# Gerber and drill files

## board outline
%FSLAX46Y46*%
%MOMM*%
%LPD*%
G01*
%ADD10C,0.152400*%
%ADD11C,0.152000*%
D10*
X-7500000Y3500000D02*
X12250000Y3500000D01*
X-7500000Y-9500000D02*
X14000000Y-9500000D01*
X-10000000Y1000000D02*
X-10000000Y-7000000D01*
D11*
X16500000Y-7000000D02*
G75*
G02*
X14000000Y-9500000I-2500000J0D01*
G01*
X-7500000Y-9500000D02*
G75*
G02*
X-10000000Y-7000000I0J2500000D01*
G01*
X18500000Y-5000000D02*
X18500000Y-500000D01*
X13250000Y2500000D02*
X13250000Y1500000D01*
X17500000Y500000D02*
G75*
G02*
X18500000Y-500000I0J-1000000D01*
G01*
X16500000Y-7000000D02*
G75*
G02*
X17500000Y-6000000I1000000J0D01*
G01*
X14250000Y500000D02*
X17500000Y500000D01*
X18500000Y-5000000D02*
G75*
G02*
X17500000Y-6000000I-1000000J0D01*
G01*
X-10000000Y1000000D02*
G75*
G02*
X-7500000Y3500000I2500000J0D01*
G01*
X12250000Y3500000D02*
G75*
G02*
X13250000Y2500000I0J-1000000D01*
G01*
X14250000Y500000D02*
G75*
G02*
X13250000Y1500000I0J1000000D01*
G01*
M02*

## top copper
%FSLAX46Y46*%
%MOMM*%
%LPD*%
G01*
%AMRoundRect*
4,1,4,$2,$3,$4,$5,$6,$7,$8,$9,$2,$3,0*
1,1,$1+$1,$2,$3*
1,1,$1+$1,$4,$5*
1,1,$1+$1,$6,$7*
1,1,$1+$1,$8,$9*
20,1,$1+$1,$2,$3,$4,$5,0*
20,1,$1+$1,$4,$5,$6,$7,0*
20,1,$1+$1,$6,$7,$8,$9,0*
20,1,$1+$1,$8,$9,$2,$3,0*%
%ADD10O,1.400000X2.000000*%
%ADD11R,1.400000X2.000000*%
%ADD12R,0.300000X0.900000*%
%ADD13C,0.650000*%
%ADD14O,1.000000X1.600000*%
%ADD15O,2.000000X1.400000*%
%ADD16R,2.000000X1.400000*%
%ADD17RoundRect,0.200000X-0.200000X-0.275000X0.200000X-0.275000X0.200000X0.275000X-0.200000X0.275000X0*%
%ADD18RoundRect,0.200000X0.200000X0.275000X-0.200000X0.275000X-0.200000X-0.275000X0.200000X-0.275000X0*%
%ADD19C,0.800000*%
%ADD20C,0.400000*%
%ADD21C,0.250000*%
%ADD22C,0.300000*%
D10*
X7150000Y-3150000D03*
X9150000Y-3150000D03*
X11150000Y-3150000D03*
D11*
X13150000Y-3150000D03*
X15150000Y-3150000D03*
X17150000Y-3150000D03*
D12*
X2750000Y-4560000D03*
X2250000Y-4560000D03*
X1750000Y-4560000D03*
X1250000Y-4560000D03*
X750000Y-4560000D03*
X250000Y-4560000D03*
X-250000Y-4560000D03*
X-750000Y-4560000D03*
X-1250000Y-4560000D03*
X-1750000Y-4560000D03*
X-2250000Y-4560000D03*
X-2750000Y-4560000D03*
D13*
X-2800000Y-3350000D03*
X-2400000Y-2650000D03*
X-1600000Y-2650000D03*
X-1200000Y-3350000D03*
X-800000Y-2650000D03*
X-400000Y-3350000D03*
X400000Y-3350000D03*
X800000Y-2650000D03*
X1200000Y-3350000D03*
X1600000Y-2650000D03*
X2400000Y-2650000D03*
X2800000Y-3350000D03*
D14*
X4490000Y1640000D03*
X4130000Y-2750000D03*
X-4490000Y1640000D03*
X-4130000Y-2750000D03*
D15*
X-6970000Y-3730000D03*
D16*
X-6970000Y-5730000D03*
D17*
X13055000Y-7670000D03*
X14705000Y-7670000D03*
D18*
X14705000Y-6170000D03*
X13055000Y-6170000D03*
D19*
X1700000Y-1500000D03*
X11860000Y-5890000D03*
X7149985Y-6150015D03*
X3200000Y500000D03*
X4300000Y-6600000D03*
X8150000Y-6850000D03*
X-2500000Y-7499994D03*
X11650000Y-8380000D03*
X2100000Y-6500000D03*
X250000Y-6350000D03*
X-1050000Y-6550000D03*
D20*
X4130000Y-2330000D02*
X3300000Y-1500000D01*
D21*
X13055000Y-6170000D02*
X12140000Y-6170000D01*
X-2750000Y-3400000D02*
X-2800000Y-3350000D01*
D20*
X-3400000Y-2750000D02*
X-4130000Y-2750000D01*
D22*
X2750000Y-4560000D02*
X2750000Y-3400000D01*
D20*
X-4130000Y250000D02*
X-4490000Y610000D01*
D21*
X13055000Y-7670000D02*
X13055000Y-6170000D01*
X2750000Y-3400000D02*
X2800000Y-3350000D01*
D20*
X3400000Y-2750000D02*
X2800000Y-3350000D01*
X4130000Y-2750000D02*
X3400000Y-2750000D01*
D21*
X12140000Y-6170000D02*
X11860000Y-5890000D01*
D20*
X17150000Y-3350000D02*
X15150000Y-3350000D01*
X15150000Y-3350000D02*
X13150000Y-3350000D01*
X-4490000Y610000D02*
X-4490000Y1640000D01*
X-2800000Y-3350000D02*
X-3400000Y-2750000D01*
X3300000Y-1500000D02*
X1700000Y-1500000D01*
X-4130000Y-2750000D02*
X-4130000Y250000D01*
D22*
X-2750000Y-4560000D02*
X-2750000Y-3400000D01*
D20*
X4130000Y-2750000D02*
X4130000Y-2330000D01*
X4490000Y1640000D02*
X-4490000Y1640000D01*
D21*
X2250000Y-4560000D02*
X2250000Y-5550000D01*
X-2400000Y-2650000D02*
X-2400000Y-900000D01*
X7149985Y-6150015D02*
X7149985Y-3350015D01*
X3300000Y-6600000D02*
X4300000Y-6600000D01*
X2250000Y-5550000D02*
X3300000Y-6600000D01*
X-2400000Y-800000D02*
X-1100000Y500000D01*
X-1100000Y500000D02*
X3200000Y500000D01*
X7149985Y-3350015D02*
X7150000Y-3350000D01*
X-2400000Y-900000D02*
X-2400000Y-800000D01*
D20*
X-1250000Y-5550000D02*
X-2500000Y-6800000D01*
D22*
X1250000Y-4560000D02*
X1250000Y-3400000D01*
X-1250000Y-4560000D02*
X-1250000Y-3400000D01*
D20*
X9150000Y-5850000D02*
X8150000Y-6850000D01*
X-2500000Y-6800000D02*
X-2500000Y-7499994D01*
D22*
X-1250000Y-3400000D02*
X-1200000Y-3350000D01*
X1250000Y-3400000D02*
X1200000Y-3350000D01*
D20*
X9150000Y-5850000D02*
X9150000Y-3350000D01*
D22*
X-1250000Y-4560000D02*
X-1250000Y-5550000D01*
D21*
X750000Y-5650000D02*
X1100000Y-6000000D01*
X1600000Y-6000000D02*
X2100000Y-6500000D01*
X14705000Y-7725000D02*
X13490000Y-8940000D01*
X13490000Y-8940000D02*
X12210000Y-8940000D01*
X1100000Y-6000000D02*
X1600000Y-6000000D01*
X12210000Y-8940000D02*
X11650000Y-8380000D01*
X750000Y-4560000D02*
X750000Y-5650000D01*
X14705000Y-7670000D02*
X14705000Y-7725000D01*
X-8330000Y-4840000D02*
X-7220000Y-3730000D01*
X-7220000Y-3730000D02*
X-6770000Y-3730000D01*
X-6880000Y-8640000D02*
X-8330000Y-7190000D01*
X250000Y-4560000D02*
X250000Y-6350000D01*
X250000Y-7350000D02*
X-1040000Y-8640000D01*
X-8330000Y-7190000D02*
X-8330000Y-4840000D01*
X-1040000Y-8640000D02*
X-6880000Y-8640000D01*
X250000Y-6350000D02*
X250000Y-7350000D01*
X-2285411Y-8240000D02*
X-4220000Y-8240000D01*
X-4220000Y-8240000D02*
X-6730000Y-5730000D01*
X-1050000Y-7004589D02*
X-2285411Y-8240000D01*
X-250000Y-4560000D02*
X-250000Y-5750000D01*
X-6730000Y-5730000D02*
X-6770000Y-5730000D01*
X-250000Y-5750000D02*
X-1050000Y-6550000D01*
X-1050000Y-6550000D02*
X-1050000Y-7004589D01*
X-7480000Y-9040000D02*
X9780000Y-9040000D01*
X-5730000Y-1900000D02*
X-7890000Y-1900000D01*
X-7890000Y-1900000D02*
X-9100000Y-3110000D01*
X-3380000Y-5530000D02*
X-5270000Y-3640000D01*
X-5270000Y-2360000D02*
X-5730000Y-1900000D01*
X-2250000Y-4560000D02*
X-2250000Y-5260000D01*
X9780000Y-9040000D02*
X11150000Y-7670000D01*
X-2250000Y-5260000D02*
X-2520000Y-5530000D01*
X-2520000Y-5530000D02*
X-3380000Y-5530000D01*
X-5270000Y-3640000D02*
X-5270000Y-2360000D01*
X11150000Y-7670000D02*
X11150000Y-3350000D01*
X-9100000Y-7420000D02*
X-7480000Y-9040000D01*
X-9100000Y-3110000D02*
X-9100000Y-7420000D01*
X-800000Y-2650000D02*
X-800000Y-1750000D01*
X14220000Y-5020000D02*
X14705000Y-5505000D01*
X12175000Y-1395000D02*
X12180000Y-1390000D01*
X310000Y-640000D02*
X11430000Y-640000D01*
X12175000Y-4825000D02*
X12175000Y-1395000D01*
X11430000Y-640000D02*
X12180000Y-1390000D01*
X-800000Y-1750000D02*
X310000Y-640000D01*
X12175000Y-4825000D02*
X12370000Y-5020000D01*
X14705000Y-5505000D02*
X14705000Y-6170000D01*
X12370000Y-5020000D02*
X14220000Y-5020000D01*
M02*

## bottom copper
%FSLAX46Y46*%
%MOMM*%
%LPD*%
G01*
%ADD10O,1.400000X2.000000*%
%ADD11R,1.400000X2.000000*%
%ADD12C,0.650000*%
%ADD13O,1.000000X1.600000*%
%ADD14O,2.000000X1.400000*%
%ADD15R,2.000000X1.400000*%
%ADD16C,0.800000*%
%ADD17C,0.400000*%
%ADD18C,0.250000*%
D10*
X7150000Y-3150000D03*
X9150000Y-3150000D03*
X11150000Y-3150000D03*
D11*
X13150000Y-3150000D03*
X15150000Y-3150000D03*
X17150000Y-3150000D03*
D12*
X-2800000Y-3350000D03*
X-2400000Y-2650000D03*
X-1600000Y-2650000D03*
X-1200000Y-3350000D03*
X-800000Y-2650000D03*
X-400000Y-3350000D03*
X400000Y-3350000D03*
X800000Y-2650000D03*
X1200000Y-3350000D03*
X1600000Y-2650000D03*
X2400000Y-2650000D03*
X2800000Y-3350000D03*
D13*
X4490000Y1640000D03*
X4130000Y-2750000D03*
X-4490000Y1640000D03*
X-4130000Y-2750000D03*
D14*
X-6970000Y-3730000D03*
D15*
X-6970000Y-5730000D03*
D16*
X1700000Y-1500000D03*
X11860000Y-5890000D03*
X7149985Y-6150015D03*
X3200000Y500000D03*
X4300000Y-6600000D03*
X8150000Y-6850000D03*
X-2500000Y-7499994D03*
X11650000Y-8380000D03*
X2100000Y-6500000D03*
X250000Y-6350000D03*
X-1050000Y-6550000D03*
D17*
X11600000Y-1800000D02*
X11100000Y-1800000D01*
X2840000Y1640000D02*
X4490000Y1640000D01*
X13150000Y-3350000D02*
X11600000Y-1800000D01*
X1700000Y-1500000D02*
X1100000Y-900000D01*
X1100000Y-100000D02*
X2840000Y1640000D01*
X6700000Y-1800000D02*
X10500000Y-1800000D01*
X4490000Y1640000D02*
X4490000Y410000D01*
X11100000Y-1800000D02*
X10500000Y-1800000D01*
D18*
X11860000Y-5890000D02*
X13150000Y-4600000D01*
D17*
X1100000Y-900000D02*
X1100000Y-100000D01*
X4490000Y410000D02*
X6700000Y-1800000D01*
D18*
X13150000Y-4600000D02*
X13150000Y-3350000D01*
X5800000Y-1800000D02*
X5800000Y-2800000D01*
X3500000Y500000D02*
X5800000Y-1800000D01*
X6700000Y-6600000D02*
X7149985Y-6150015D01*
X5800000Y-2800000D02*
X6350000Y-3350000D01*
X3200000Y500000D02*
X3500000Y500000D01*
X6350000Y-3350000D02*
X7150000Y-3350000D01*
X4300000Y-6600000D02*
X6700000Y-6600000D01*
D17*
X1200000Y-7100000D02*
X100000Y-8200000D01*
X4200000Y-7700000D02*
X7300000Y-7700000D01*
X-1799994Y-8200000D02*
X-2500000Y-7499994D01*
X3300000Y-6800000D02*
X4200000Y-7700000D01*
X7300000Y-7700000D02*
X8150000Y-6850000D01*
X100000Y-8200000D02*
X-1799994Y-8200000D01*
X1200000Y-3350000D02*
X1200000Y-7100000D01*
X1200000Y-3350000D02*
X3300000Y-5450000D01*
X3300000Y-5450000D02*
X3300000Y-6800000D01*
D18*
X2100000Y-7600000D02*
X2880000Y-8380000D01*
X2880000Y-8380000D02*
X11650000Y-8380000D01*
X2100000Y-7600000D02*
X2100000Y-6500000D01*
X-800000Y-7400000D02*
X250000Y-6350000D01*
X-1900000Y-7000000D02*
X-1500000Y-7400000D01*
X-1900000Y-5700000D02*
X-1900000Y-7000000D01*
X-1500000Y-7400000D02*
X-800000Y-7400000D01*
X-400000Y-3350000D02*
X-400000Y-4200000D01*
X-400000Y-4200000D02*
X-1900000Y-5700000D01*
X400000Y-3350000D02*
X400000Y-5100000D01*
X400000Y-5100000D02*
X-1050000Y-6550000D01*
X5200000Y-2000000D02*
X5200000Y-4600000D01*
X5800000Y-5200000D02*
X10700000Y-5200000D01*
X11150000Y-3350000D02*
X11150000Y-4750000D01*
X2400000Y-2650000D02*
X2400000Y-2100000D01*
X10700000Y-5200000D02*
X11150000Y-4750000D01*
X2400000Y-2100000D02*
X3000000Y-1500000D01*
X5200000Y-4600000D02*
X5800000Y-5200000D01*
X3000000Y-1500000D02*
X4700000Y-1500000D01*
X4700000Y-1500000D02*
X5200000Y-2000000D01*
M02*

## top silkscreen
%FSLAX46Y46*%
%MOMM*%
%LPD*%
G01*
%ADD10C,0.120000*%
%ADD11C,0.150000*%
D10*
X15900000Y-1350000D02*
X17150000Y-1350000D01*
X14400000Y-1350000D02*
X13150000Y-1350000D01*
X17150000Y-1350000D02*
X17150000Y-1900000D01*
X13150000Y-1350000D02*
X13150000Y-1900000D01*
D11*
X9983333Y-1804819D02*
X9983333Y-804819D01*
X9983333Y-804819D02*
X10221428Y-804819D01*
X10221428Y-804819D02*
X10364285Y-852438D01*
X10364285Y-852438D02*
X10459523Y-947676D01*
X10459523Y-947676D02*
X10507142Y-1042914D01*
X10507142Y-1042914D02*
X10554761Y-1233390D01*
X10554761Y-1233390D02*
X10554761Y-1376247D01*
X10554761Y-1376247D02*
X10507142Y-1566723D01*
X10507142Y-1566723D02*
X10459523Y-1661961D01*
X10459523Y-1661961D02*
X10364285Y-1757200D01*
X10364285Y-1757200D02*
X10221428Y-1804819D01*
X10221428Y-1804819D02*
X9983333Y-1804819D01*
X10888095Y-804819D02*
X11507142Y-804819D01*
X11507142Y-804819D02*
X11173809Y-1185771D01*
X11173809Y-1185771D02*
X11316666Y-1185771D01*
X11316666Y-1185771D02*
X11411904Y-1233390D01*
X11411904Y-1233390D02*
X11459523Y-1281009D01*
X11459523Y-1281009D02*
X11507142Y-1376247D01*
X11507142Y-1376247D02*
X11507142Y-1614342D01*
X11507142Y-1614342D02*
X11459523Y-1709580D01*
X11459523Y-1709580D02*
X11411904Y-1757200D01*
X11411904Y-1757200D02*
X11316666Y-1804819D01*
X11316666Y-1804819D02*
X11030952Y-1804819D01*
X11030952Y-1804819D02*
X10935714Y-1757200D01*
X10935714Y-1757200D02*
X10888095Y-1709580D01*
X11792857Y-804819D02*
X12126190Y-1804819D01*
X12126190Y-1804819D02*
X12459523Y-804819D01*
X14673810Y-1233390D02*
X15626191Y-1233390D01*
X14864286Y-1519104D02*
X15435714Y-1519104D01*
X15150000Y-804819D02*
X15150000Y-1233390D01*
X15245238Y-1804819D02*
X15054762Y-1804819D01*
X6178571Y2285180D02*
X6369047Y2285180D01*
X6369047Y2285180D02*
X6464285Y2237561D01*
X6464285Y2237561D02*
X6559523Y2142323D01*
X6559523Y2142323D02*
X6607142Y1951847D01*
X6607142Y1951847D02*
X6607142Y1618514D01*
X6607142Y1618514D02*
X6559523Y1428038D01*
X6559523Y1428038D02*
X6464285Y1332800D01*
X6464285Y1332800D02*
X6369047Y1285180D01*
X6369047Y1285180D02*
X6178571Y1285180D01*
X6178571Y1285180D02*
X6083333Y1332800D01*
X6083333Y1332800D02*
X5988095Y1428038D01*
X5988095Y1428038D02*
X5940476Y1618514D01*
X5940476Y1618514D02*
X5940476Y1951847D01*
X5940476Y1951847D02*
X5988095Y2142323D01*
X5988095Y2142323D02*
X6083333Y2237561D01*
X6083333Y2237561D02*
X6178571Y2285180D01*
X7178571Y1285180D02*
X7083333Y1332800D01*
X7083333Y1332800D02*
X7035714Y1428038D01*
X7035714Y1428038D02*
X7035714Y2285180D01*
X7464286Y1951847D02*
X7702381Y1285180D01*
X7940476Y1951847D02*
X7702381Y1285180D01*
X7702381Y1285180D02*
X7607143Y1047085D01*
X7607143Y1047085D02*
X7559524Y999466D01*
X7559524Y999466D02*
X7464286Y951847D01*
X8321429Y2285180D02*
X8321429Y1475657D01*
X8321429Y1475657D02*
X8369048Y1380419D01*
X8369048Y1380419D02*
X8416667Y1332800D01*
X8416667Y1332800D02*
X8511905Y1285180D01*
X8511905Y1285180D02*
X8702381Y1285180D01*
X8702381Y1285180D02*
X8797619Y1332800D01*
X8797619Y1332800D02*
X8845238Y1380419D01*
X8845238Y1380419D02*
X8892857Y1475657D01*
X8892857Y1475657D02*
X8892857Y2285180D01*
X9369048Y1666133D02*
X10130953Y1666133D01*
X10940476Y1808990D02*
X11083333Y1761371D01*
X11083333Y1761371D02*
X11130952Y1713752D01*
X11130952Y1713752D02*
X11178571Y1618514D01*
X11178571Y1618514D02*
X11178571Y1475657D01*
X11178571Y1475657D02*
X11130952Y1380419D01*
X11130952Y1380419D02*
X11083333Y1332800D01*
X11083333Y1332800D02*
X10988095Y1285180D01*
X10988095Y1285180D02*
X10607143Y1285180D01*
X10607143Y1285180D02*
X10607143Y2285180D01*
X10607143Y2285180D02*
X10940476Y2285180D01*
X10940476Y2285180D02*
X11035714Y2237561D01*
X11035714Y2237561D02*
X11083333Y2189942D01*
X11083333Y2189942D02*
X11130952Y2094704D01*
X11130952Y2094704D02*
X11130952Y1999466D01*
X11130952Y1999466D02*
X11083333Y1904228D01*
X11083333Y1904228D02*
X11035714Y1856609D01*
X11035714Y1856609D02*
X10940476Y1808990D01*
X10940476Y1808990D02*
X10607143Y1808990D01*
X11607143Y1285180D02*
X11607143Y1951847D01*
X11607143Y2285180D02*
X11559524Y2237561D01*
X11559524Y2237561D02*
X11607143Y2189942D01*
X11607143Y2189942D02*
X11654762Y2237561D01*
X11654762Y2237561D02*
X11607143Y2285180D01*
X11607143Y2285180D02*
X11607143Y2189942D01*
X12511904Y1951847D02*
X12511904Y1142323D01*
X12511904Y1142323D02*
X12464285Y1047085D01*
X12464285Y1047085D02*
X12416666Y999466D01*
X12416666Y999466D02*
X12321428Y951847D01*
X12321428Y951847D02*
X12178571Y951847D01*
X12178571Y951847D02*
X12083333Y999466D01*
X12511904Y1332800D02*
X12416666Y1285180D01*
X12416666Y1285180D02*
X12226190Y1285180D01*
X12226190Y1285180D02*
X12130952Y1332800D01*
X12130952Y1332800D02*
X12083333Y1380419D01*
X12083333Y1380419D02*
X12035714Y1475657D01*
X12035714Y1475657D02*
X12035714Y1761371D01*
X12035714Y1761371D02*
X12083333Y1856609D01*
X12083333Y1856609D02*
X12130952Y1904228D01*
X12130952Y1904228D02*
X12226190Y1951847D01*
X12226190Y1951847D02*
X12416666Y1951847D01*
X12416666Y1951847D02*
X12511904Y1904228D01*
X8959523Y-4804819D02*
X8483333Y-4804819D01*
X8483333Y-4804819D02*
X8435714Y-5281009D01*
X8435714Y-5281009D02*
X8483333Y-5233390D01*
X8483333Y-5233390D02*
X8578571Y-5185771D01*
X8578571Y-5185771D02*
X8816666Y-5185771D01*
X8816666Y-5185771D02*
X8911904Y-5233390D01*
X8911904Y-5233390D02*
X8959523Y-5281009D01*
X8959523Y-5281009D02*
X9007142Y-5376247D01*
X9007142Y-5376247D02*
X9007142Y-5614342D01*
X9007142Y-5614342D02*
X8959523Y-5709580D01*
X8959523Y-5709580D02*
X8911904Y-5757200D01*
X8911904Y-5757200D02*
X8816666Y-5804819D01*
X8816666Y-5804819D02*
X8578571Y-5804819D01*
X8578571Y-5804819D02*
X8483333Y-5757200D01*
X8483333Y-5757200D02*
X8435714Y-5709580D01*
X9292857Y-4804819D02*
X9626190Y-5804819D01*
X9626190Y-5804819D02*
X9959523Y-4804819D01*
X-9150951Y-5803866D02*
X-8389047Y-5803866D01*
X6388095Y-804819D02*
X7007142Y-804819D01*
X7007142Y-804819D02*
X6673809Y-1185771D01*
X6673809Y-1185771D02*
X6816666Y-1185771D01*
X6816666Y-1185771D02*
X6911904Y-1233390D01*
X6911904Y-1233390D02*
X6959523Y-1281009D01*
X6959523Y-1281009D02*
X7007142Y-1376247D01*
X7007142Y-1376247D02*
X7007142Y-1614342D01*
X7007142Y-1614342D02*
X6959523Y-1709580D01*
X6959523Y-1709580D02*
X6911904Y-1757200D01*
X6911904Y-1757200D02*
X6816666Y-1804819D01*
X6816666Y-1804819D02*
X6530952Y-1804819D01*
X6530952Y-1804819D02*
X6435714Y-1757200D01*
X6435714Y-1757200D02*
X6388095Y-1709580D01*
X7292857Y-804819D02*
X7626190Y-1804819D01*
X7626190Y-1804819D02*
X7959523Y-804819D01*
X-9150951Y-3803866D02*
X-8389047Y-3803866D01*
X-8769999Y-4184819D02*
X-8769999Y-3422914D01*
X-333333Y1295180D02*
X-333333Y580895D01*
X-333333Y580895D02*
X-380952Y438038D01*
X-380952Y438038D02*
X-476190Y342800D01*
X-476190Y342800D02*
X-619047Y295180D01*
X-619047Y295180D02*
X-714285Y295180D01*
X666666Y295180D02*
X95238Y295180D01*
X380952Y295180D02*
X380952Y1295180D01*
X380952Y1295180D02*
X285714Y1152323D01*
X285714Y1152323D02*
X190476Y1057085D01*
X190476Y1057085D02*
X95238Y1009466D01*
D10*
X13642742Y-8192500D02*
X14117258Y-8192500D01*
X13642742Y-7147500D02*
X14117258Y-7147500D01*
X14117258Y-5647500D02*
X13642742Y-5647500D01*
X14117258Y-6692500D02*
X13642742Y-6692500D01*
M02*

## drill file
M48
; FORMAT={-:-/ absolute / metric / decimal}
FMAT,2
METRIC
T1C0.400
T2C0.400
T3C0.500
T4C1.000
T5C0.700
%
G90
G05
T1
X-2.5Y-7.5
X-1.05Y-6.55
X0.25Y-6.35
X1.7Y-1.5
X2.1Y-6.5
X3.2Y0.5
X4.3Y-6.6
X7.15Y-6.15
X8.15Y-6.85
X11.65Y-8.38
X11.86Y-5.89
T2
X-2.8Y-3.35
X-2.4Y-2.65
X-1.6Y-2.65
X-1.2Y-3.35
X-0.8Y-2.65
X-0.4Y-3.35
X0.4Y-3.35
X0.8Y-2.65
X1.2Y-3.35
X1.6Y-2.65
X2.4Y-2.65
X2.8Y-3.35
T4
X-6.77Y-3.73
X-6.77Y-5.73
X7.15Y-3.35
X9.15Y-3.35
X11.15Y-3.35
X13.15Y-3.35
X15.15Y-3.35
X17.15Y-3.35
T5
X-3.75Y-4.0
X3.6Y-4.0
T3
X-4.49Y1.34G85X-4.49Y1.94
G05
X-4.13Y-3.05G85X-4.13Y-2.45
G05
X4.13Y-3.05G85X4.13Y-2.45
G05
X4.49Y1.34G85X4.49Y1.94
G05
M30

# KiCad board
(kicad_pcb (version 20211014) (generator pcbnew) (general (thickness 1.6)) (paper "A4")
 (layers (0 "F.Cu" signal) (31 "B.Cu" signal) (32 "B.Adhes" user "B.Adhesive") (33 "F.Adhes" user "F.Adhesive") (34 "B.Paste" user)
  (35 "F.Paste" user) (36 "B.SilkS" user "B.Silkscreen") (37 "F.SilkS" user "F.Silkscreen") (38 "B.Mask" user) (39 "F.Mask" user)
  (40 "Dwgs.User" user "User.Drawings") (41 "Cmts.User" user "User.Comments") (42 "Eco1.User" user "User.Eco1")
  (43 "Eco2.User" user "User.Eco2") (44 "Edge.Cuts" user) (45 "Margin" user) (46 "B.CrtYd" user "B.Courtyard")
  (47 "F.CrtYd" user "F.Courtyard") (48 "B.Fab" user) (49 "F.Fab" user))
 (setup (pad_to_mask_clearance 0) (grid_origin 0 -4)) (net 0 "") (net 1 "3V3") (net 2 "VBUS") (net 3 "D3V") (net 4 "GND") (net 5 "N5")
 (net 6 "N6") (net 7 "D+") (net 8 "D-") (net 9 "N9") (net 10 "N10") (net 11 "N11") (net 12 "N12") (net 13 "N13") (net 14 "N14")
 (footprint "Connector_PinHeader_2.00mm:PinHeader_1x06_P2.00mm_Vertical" (layer "F.Cu") (at 7.15 3.35 90)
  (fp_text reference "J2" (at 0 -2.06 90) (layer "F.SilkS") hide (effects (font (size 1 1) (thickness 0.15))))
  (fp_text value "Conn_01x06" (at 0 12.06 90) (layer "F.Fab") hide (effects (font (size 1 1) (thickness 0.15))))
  (pad "1" thru_hole oval locked (at 0 0 90) (size 2 1.4) (drill 1 (offset 0.2 0)) (layers *.Cu *.Mask) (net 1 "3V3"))
  (pad "2" thru_hole oval locked (at 0 2 90) (size 2 1.4) (drill 1 (offset 0.2 0)) (layers *.Cu *.Mask) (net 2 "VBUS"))
  (pad "3" thru_hole oval locked (at 0 4 90) (size 2 1.4) (drill 1 (offset 0.2 0)) (layers *.Cu *.Mask) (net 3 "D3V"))
  (pad "4" thru_hole rect locked (at 0 6 90) (size 2 1.4) (drill 1 (offset 0.2 0)) (layers *.Cu *.Mask) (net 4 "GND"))
  (pad "5" thru_hole rect locked (at 0 8 90) (size 2 1.4) (drill 1 (offset 0.2 0)) (layers *.Cu *.Mask) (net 4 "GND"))
  (pad "6" thru_hole rect locked (at 0 10 90) (size 2 1.4) (drill 1 (offset 0.2 0)) (layers *.Cu *.Mask) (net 4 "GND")))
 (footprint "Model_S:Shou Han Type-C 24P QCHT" (layer "F.Cu") (at 0 -3.5 180)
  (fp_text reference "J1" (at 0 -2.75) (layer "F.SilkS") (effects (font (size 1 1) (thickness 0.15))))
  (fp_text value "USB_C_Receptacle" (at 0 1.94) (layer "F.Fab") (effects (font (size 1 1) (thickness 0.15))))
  (pad "" np_thru_hole circle locked (at -3.6 -7.5 180) (size 0.7 0.7) (drill 0.7) (layers *.Cu *.Mask))
  (pad "" np_thru_hole circle locked (at 3.75 -7.5 180) (size 0.7 0.7) (drill 0.7) (layers *.Cu *.Mask))
  (pad "A1" smd rect locked (at -2.75 -8.06 180) (size 0.3 0.9) (layers "F.Cu" "F.Paste" "F.Mask") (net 4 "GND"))
  (pad "A2" smd rect locked (at -2.25 -8.06 180) (size 0.3 0.9) (layers "F.Cu" "F.Paste" "F.Mask") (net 1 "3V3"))
  (pad "A3" smd rect locked (at -1.75 -8.06 180) (size 0.3 0.9) (layers "F.Cu" "F.Paste" "F.Mask") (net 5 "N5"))
  (pad "A4" smd rect locked (at -1.25 -8.06 180) (size 0.3 0.9) (layers "F.Cu" "F.Paste" "F.Mask") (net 2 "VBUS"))
  (pad "A5" smd rect locked (at -0.75 -8.06 180) (size 0.3 0.9) (layers "F.Cu" "F.Paste" "F.Mask") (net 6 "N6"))
  (pad "A6" smd rect locked (at -0.25 -8.06 180) (size 0.3 0.9) (layers "F.Cu" "F.Paste" "F.Mask") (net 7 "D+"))
  (pad "A7" smd rect locked (at 0.25 -8.06 180) (size 0.3 0.9) (layers "F.Cu" "F.Paste" "F.Mask") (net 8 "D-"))
  (pad "A8" smd rect locked (at 0.75 -8.06 180) (size 0.3 0.9) (layers "F.Cu" "F.Paste" "F.Mask") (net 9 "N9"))
  (pad "A9" smd rect locked (at 1.25 -8.06 180) (size 0.3 0.9) (layers "F.Cu" "F.Paste" "F.Mask") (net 2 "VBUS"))
  (pad "A10" smd rect locked (at 1.75 -8.06 180) (size 0.3 0.9) (layers "F.Cu" "F.Paste" "F.Mask") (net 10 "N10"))
  (pad "A11" smd rect locked (at 2.25 -8.06 180) (size 0.3 0.9) (layers "F.Cu" "F.Paste" "F.Mask") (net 3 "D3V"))
  (pad "A12" smd rect locked (at 2.75 -8.06 180) (size 0.3 0.9) (layers "F.Cu" "F.Paste" "F.Mask") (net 4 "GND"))
  (pad "B1" thru_hole circle locked (at 2.8 -6.85 180) (size 0.65 0.65) (drill 0.4) (layers *.Cu *.Mask) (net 4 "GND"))
  (pad "B2" thru_hole circle locked (at 2.4 -6.15 180) (size 0.65 0.65) (drill 0.4) (layers *.Cu *.Mask) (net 1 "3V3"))
  (pad "B3" thru_hole circle locked (at 1.6 -6.15 180) (size 0.65 0.65) (drill 0.4) (layers *.Cu *.Mask) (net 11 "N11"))
  (pad "B4" thru_hole circle locked (at 1.2 -6.85 180) (size 0.65 0.65) (drill 0.4) (layers *.Cu *.Mask) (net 2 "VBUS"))
  (pad "B5" thru_hole circle locked (at 0.8 -6.15 180) (size 0.65 0.65) (drill 0.4) (layers *.Cu *.Mask) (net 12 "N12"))
  (pad "B6" thru_hole circle locked (at 0.4 -6.85 180) (size 0.65 0.65) (drill 0.4) (layers *.Cu *.Mask) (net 7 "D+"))
  (pad "B7" thru_hole circle locked (at -0.4 -6.85 180) (size 0.65 0.65) (drill 0.4) (layers *.Cu *.Mask) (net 8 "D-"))
  (pad "B8" thru_hole circle locked (at -0.8 -6.15 180) (size 0.65 0.65) (drill 0.4) (layers *.Cu *.Mask) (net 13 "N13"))
  (pad "B9" thru_hole circle locked (at -1.2 -6.85 180) (size 0.65 0.65) (drill 0.4) (layers *.Cu *.Mask) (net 2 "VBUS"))
  (pad "B10" thru_hole circle locked (at -1.6 -6.15 180) (size 0.65 0.65) (drill 0.4) (layers *.Cu *.Mask) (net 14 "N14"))
  (pad "B11" thru_hole circle locked (at -2.4 -6.15 180) (size 0.65 0.65) (drill 0.4) (layers *.Cu *.Mask) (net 3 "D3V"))
  (pad "B12" thru_hole circle locked (at -2.8 -6.85 180) (size 0.65 0.65) (drill 0.4) (layers *.Cu *.Mask) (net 4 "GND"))
  (pad "S1" thru_hole oval locked (at -4.49 -1.86 180) (size 1 1.6) (drill oval 0.5 1.1) (layers *.Cu *.Mask) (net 4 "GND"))
  (pad "S1" thru_hole oval locked (at -4.13 -6.25 180) (size 1 1.6) (drill oval 0.5 1.1) (layers *.Cu *.Mask) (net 4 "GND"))
  (pad "S1" thru_hole oval locked (at 4.49 -1.86 180) (size 1 1.6) (drill oval 0.5 1.1) (layers *.Cu *.Mask) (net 4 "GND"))
  (pad "S1" thru_hole oval locked (at 4.13 -6.25 180) (size 1 1.6) (drill oval 0.5 1.1) (layers *.Cu *.Mask) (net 4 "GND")))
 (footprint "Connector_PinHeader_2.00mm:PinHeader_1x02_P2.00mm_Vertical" (layer "F.Cu") (at -6.77 3.73)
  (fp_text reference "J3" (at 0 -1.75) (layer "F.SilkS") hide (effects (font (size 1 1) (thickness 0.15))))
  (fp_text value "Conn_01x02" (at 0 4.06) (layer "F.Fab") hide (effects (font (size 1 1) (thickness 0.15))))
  (pad "1" thru_hole oval locked (at 0 0) (size 2 1.4) (drill 1 (offset -0.2 0)) (layers *.Cu *.Mask) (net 7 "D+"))
  (pad "2" thru_hole rect locked (at 0 2) (size 2 1.4) (drill 1 (offset -0.2 0)) (layers *.Cu *.Mask) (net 8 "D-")))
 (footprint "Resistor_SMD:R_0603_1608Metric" (layer "F.Cu") (at 13.88 7.67)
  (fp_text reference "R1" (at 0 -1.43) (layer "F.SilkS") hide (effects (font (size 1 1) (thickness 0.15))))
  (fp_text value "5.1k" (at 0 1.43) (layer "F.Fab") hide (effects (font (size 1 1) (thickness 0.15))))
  (fp_line (start -0.237258 0.5225) (end 0.237258 0.5225) (layer "F.SilkS") (width 0.12))
  (fp_line (start -0.237258 -0.5225) (end 0.237258 -0.5225) (layer "F.SilkS") (width 0.12))
  (pad "1" smd roundrect locked (at -0.825 0) (size 0.8 0.95) (layers "F.Cu" "F.Paste" "F.Mask") (roundrect_rratio 0.25) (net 4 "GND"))
  (pad "2" smd roundrect locked (at 0.825 0) (size 0.8 0.95) (layers "F.Cu" "F.Paste" "F.Mask") (roundrect_rratio 0.25) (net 6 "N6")))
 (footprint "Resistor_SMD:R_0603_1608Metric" (layer "F.Cu") (at 13.88 6.17 180)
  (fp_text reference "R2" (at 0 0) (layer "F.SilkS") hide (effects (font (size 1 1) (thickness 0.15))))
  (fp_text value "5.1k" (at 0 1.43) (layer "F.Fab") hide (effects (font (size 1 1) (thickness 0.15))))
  (fp_line (start -0.237258 0.5225) (end 0.237258 0.5225) (layer "F.SilkS") (width 0.12))
  (fp_line (start -0.237258 -0.5225) (end 0.237258 -0.5225) (layer "F.SilkS") (width 0.12))
  (pad "1" smd roundrect locked (at -0.825 0 180) (size 0.8 0.95) (layers "F.Cu" "F.Paste" "F.Mask") (roundrect_rratio 0.25) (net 12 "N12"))
  (pad "2" smd roundrect locked (at 0.825 0 180) (size 0.8 0.95) (layers "F.Cu" "F.Paste" "F.Mask") (roundrect_rratio 0.25) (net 4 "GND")))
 (gr_line (start 15.9 1.35) (end 17.15 1.35) (layer "F.SilkS") (width 0.12))
 (gr_line (start 14.4 1.35) (end 13.15 1.35) (layer "F.SilkS") (width 0.12))
 (gr_line (start 17.15 1.35) (end 17.15 1.9) (layer "F.SilkS") (width 0.12))
 (gr_line (start 13.15 1.35) (end 13.15 1.9) (layer "F.SilkS") (width 0.12))
 (gr_line (start -7.5 -3.5) (end 12.25 -3.5) (layer "Edge.Cuts") (width 0.1524))
 (gr_line (start -7.5 9.5) (end 14 9.5) (layer "Edge.Cuts") (width 0.1524))
 (gr_line (start -10 -1) (end -10 7) (layer "Edge.Cuts") (width 0.1524))
 (gr_arc (start 16.5 7) (mid 15.767767 8.767767) (end 14 9.5) (layer "Edge.Cuts") (width 0.152))
 (gr_arc (start -7.5 9.5) (mid -9.267767 8.767767) (end -10 7) (layer "Edge.Cuts") (width 0.152))
 (gr_line (start 18.5 5) (end 18.5 0.5) (layer "Edge.Cuts") (width 0.152))
 (gr_line (start 13.25 -2.5) (end 13.25 -1.5) (layer "Edge.Cuts") (width 0.152))
 (gr_arc (start 17.5 -0.5) (mid 18.207107 -0.207107) (end 18.5 0.5) (layer "Edge.Cuts") (width 0.152))
 (gr_arc (start 16.5 7) (mid 16.792893 6.292893) (end 17.5 6) (layer "Edge.Cuts") (width 0.152))
 (gr_line (start 14.25 -0.5) (end 17.5 -0.5) (layer "Edge.Cuts") (width 0.152))
 (gr_arc (start 18.5 5) (mid 18.207107 5.707107) (end 17.5 6) (layer "Edge.Cuts") (width 0.152))
 (gr_arc (start -10 -1) (mid -9.267767 -2.767767) (end -7.5 -3.5) (layer "Edge.Cuts") (width 0.152))
 (gr_arc (start 12.25 -3.5) (mid 12.957107 -3.207107) (end 13.25 -2.5) (layer "Edge.Cuts") (width 0.152))
 (gr_arc (start 14.25 -0.5) (mid 13.542893 -0.792893) (end 13.25 -1.5) (layer "Edge.Cuts") (width 0.152))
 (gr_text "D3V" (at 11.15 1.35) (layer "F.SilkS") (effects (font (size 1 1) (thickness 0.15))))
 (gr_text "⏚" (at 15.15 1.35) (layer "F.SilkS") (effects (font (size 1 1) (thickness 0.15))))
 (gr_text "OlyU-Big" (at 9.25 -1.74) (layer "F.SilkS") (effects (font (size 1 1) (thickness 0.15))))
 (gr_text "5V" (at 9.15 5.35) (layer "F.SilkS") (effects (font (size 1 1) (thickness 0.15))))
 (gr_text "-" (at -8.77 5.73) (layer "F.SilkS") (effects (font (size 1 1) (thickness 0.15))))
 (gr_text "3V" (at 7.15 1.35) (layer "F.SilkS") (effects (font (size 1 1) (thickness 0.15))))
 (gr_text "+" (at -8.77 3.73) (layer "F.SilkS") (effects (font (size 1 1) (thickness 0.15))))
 (segment (start 4.13 2.33) (end 3.3 1.5) (width 0.4) (layer "F.Cu") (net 4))
 (segment (start 13.055 6.17) (end 12.14 6.17) (width 0.25) (layer "F.Cu") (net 4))
 (segment (start -2.75 3.4) (end -2.8 3.35) (width 0.25) (layer "F.Cu") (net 4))
 (segment (start -3.4 2.75) (end -4.13 2.75) (width 0.4) (layer "F.Cu") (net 4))
 (segment (start 2.75 4.56) (end 2.75 3.4) (width 0.3) (layer "F.Cu") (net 4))
 (segment (start -4.13 -0.25) (end -4.49 -0.61) (width 0.4) (layer "F.Cu") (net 4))
 (segment (start 13.055 7.67) (end 13.055 6.17) (width 0.25) (layer "F.Cu") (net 4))
 (segment (start 2.75 3.4) (end 2.8 3.35) (width 0.25) (layer "F.Cu") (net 4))
 (segment (start 3.4 2.75) (end 2.8 3.35) (width 0.4) (layer "F.Cu") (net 4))
 (segment (start 4.13 2.75) (end 3.4 2.75) (width 0.4) (layer "F.Cu") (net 4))
 (segment (start 12.14 6.17) (end 11.86 5.89) (width 0.25) (layer "F.Cu") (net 4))
 (segment (start 17.15 3.35) (end 15.15 3.35) (width 0.4) (layer "F.Cu") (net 4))
 (segment (start 15.15 3.35) (end 13.15 3.35) (width 0.4) (layer "F.Cu") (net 4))
 (segment (start -4.49 -0.61) (end -4.49 -1.64) (width 0.4) (layer "F.Cu") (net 4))
 (segment (start -2.8 3.35) (end -3.4 2.75) (width 0.4) (layer "F.Cu") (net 4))
 (segment (start 3.3 1.5) (end 1.7 1.5) (width 0.4) (layer "F.Cu") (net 4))
 (segment (start -4.13 2.75) (end -4.13 -0.25) (width 0.4) (layer "F.Cu") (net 4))
 (segment (start -2.75 4.56) (end -2.75 3.4) (width 0.3) (layer "F.Cu") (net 4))
 (segment (start 4.13 2.75) (end 4.13 2.33) (width 0.4) (layer "F.Cu") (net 4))
 (segment (start 4.49 -1.64) (end -4.49 -1.64) (width 0.4) (layer "F.Cu") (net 4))
 (via (at 1.7 1.5) (size 0.8) (drill 0.4) (layers "F.Cu" "B.Cu") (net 4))
 (via (at 11.86 5.89) (size 0.8) (drill 0.4) (layers "F.Cu" "B.Cu") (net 4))
 (segment (start 11.6 1.8) (end 11.1 1.8) (width 0.4) (layer "B.Cu") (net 4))
 (segment (start 2.84 -1.64) (end 4.49 -1.64) (width 0.4) (layer "B.Cu") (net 4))
 (segment (start 13.15 3.35) (end 11.6 1.8) (width 0.4) (layer "B.Cu") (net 4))
 (segment (start 1.7 1.5) (end 1.1 0.9) (width 0.4) (layer "B.Cu") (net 4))
 (segment (start 1.1 0.1) (end 2.84 -1.64) (width 0.4) (layer "B.Cu") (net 4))
 (segment (start 6.7 1.8) (end 10.5 1.8) (width 0.4) (layer "B.Cu") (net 4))
 (segment (start 4.49 -1.64) (end 4.49 -0.41) (width 0.4) (layer "B.Cu") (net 4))
 (segment (start 11.1 1.8) (end 10.5 1.8) (width 0.4) (layer "B.Cu") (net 4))
 (segment (start 11.86 5.89) (end 13.15 4.6) (width 0.25) (layer "B.Cu") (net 4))
 (segment (start 1.1 0.9) (end 1.1 0.1) (width 0.4) (layer "B.Cu") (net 4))
 (segment (start 4.49 -0.41) (end 6.7 1.8) (width 0.4) (layer "B.Cu") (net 4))
 (segment (start 13.15 4.6) (end 13.15 3.35) (width 0.25) (layer "B.Cu") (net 4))
 (segment (start 2.25 4.56) (end 2.25 5.55) (width 0.25) (layer "F.Cu") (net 1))
 (segment (start -2.4 2.65) (end -2.4 0.9) (width 0.25) (layer "F.Cu") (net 1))
 (segment (start 7.149985 6.150015) (end 7.149985 3.350015) (width 0.25) (layer "F.Cu") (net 1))
 (segment (start 3.3 6.6) (end 4.3 6.6) (width 0.25) (layer "F.Cu") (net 1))
 (segment (start 2.25 5.55) (end 3.3 6.6) (width 0.25) (layer "F.Cu") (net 1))
 (segment (start -2.4 0.8) (end -1.1 -0.5) (width 0.25) (layer "F.Cu") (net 1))
 (segment (start -1.1 -0.5) (end 3.2 -0.5) (width 0.25) (layer "F.Cu") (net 1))
 (segment (start 7.149985 3.350015) (end 7.15 3.35) (width 0.25) (layer "F.Cu") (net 1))
 (segment (start -2.4 0.9) (end -2.4 0.8) (width 0.25) (layer "F.Cu") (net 1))
 (via (at 7.149985 6.150015) (size 0.8) (drill 0.4) (layers "F.Cu" "B.Cu") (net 1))
 (via (at 3.2 -0.5) (size 0.8) (drill 0.4) (layers "F.Cu" "B.Cu") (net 1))
 (via (at 4.3 6.6) (size 0.8) (drill 0.4) (layers "F.Cu" "B.Cu") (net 1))
 (segment (start 5.8 1.8) (end 5.8 2.8) (width 0.25) (layer "B.Cu") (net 1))
 (segment (start 3.5 -0.5) (end 5.8 1.8) (width 0.25) (layer "B.Cu") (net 1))
 (segment (start 6.7 6.6) (end 7.149985 6.150015) (width 0.25) (layer "B.Cu") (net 1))
 (segment (start 5.8 2.8) (end 6.35 3.35) (width 0.25) (layer "B.Cu") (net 1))
 (segment (start 3.2 -0.5) (end 3.5 -0.5) (width 0.25) (layer "B.Cu") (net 1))
 (segment (start 6.35 3.35) (end 7.15 3.35) (width 0.25) (layer "B.Cu") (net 1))
 (segment (start 4.3 6.6) (end 6.7 6.6) (width 0.25) (layer "B.Cu") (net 1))
 (segment (start -1.25 5.55) (end -2.5 6.8) (width 0.4) (layer "F.Cu") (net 2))
 (segment (start 1.25 4.56) (end 1.25 3.4) (width 0.3) (layer "F.Cu") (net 2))
 (segment (start -1.25 4.56) (end -1.25 3.4) (width 0.3) (layer "F.Cu") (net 2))
 (segment (start 9.15 5.85) (end 8.15 6.85) (width 0.4) (layer "F.Cu") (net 2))
 (segment (start -2.5 6.8) (end -2.5 7.499994) (width 0.4) (layer "F.Cu") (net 2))
 (segment (start -1.25 3.4) (end -1.2 3.35) (width 0.3) (layer "F.Cu") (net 2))
 (segment (start 1.25 3.4) (end 1.2 3.35) (width 0.3) (layer "F.Cu") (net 2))
 (segment (start 9.15 5.85) (end 9.15 3.35) (width 0.4) (layer "F.Cu") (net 2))
 (segment (start -1.25 4.56) (end -1.25 5.55) (width 0.3) (layer "F.Cu") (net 2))
 (via (at 8.15 6.85) (size 0.8) (drill 0.4) (layers "F.Cu" "B.Cu") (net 2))
 (via (at -2.5 7.499994) (size 0.8) (drill 0.4) (layers "F.Cu" "B.Cu") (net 2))
 (segment (start 1.2 7.1) (end 0.1 8.2) (width 0.4) (layer "B.Cu") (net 2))
 (segment (start 4.2 7.7) (end 7.3 7.7) (width 0.4) (layer "B.Cu") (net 2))
 (segment (start -1.799994 8.2) (end -2.5 7.499994) (width 0.4) (layer "B.Cu") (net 2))
 (segment (start 3.3 6.8) (end 4.2 7.7) (width 0.4) (layer "B.Cu") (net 2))
 (segment (start 7.3 7.7) (end 8.15 6.85) (width 0.4) (layer "B.Cu") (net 2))
 (segment (start 0.1 8.2) (end -1.799994 8.2) (width 0.4) (layer "B.Cu") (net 2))
 (segment (start 1.2 3.35) (end 1.2 7.1) (width 0.4) (layer "B.Cu") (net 2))
 (segment (start 1.2 3.35) (end 3.3 5.45) (width 0.4) (layer "B.Cu") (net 2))
 (segment (start 3.3 5.45) (end 3.3 6.8) (width 0.4) (layer "B.Cu") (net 2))
 (segment (start 0.75 5.65) (end 1.1 6) (width 0.25) (layer "F.Cu") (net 6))
 (segment (start 1.6 6) (end 2.1 6.5) (width 0.25) (layer "F.Cu") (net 6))
 (segment (start 14.705 7.725) (end 13.49 8.94) (width 0.25) (layer "F.Cu") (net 6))
 (segment (start 13.49 8.94) (end 12.21 8.94) (width 0.25) (layer "F.Cu") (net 6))
 (segment (start 1.1 6) (end 1.6 6) (width 0.25) (layer "F.Cu") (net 6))
 (segment (start 12.21 8.94) (end 11.65 8.38) (width 0.25) (layer "F.Cu") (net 6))
 (segment (start 0.75 4.56) (end 0.75 5.65) (width 0.25) (layer "F.Cu") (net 6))
 (segment (start 14.705 7.67) (end 14.705 7.725) (width 0.25) (layer "F.Cu") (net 6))
 (via (at 11.65 8.38) (size 0.8) (drill 0.4) (layers "F.Cu" "B.Cu") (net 6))
 (via (at 2.1 6.5) (size 0.8) (drill 0.4) (layers "F.Cu" "B.Cu") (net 6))
 (segment (start 2.1 7.6) (end 2.88 8.38) (width 0.25) (layer "B.Cu") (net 6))
 (segment (start 2.88 8.38) (end 11.65 8.38) (width 0.25) (layer "B.Cu") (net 6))
 (segment (start 2.1 7.6) (end 2.1 6.5) (width 0.25) (layer "B.Cu") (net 6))
 (segment (start -8.33 4.84) (end -7.22 3.73) (width 0.25) (layer "F.Cu") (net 7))
 (segment (start -7.22 3.73) (end -6.77 3.73) (width 0.25) (layer "F.Cu") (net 7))
 (segment (start -6.88 8.64) (end -8.33 7.19) (width 0.25) (layer "F.Cu") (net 7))
 (segment (start 0.25 4.56) (end 0.25 6.35) (width 0.25) (layer "F.Cu") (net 7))
 (segment (start 0.25 7.35) (end -1.04 8.64) (width 0.25) (layer "F.Cu") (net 7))
 (segment (start -8.33 7.19) (end -8.33 4.84) (width 0.25) (layer "F.Cu") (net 7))
 (segment (start -1.04 8.64) (end -6.88 8.64) (width 0.25) (layer "F.Cu") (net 7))
 (segment (start 0.25 6.35) (end 0.25 7.35) (width 0.25) (layer "F.Cu") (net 7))
 (via (at 0.25 6.35) (size 0.8) (drill 0.4) (layers "F.Cu" "B.Cu") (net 7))
 (segment (start -0.8 7.4) (end 0.25 6.35) (width 0.25) (layer "B.Cu") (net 7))
 (segment (start -1.9 7) (end -1.5 7.4) (width 0.25) (layer "B.Cu") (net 7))
 (segment (start -1.9 5.7) (end -1.9 7) (width 0.25) (layer "B.Cu") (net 7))
 (segment (start -1.5 7.4) (end -0.8 7.4) (width 0.25) (layer "B.Cu") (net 7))
 (segment (start -0.4 3.35) (end -0.4 4.2) (width 0.25) (layer "B.Cu") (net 7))
 (segment (start -0.4 4.2) (end -1.9 5.7) (width 0.25) (layer "B.Cu") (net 7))
 (segment (start -2.285411 8.24) (end -4.22 8.24) (width 0.25) (layer "F.Cu") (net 8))
 (segment (start -4.22 8.24) (end -6.73 5.73) (width 0.25) (layer "F.Cu") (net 8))
 (segment (start -1.05 7.004589) (end -2.285411 8.24) (width 0.25) (layer "F.Cu") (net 8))
 (segment (start -0.25 4.56) (end -0.25 5.75) (width 0.25) (layer "F.Cu") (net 8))
 (segment (start -6.73 5.73) (end -6.77 5.73) (width 0.25) (layer "F.Cu") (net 8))
 (segment (start -0.25 5.75) (end -1.05 6.55) (width 0.25) (layer "F.Cu") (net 8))
 (segment (start -1.05 6.55) (end -1.05 7.004589) (width 0.25) (layer "F.Cu") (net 8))
 (via (at -1.05 6.55) (size 0.8) (drill 0.4) (layers "F.Cu" "B.Cu") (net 8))
 (segment (start 0.4 3.35) (end 0.4 5.1) (width 0.25) (layer "B.Cu") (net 8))
 (segment (start 0.4 5.1) (end -1.05 6.55) (width 0.25) (layer "B.Cu") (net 8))
 (segment (start -7.48 9.04) (end 9.78 9.04) (width 0.25) (layer "F.Cu") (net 3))
 (segment (start -5.73 1.9) (end -7.89 1.9) (width 0.25) (layer "F.Cu") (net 3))
 (segment (start -7.89 1.9) (end -9.1 3.11) (width 0.25) (layer "F.Cu") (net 3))
 (segment (start -3.38 5.53) (end -5.27 3.64) (width 0.25) (layer "F.Cu") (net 3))
 (segment (start -5.27 2.36) (end -5.73 1.9) (width 0.25) (layer "F.Cu") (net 3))
 (segment (start -2.25 4.56) (end -2.25 5.26) (width 0.25) (layer "F.Cu") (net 3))
 (segment (start 9.78 9.04) (end 11.15 7.67) (width 0.25) (layer "F.Cu") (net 3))
 (segment (start -2.25 5.26) (end -2.52 5.53) (width 0.25) (layer "F.Cu") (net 3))
 (segment (start -2.52 5.53) (end -3.38 5.53) (width 0.25) (layer "F.Cu") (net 3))
 (segment (start -5.27 3.64) (end -5.27 2.36) (width 0.25) (layer "F.Cu") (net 3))
 (segment (start 11.15 7.67) (end 11.15 3.35) (width 0.25) (layer "F.Cu") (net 3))
 (segment (start -9.1 7.42) (end -7.48 9.04) (width 0.25) (layer "F.Cu") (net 3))
 (segment (start -9.1 3.11) (end -9.1 7.42) (width 0.25) (layer "F.Cu") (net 3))
 (segment (start 5.2 2) (end 5.2 4.6) (width 0.25) (layer "B.Cu") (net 3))
 (segment (start 5.8 5.2) (end 10.7 5.2) (width 0.25) (layer "B.Cu") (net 3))
 (segment (start 11.15 3.35) (end 11.15 4.75) (width 0.25) (layer "B.Cu") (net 3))
 (segment (start 2.4 2.65) (end 2.4 2.1) (width 0.25) (layer "B.Cu") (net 3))
 (segment (start 10.7 5.2) (end 11.15 4.75) (width 0.25) (layer "B.Cu") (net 3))
 (segment (start 2.4 2.1) (end 3 1.5) (width 0.25) (layer "B.Cu") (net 3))
 (segment (start 5.2 4.6) (end 5.8 5.2) (width 0.25) (layer "B.Cu") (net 3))
 (segment (start 3 1.5) (end 4.7 1.5) (width 0.25) (layer "B.Cu") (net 3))
 (segment (start 4.7 1.5) (end 5.2 2) (width 0.25) (layer "B.Cu") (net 3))
 (segment (start -0.8 2.65) (end -0.8 1.75) (width 0.25) (layer "F.Cu") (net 12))
 (segment (start 14.22 5.02) (end 14.705 5.505) (width 0.25) (layer "F.Cu") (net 12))
 (segment (start 12.175 1.395) (end 12.18 1.39) (width 0.25) (layer "F.Cu") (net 12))
 (segment (start 0.31 0.64) (end 11.43 0.64) (width 0.25) (layer "F.Cu") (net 12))
 (segment (start 12.175 4.825) (end 12.175 1.395) (width 0.25) (layer "F.Cu") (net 12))
 (segment (start 11.43 0.64) (end 12.18 1.39) (width 0.25) (layer "F.Cu") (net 12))
 (segment (start -0.8 1.75) (end 0.31 0.64) (width 0.25) (layer "F.Cu") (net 12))
 (segment (start 12.175 4.825) (end 12.37 5.02) (width 0.25) (layer "F.Cu") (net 12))
 (segment (start 14.705 5.505) (end 14.705 6.17) (width 0.25) (layer "F.Cu") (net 12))
 (segment (start 12.37 5.02) (end 14.22 5.02) (width 0.25) (layer "F.Cu") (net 12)))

